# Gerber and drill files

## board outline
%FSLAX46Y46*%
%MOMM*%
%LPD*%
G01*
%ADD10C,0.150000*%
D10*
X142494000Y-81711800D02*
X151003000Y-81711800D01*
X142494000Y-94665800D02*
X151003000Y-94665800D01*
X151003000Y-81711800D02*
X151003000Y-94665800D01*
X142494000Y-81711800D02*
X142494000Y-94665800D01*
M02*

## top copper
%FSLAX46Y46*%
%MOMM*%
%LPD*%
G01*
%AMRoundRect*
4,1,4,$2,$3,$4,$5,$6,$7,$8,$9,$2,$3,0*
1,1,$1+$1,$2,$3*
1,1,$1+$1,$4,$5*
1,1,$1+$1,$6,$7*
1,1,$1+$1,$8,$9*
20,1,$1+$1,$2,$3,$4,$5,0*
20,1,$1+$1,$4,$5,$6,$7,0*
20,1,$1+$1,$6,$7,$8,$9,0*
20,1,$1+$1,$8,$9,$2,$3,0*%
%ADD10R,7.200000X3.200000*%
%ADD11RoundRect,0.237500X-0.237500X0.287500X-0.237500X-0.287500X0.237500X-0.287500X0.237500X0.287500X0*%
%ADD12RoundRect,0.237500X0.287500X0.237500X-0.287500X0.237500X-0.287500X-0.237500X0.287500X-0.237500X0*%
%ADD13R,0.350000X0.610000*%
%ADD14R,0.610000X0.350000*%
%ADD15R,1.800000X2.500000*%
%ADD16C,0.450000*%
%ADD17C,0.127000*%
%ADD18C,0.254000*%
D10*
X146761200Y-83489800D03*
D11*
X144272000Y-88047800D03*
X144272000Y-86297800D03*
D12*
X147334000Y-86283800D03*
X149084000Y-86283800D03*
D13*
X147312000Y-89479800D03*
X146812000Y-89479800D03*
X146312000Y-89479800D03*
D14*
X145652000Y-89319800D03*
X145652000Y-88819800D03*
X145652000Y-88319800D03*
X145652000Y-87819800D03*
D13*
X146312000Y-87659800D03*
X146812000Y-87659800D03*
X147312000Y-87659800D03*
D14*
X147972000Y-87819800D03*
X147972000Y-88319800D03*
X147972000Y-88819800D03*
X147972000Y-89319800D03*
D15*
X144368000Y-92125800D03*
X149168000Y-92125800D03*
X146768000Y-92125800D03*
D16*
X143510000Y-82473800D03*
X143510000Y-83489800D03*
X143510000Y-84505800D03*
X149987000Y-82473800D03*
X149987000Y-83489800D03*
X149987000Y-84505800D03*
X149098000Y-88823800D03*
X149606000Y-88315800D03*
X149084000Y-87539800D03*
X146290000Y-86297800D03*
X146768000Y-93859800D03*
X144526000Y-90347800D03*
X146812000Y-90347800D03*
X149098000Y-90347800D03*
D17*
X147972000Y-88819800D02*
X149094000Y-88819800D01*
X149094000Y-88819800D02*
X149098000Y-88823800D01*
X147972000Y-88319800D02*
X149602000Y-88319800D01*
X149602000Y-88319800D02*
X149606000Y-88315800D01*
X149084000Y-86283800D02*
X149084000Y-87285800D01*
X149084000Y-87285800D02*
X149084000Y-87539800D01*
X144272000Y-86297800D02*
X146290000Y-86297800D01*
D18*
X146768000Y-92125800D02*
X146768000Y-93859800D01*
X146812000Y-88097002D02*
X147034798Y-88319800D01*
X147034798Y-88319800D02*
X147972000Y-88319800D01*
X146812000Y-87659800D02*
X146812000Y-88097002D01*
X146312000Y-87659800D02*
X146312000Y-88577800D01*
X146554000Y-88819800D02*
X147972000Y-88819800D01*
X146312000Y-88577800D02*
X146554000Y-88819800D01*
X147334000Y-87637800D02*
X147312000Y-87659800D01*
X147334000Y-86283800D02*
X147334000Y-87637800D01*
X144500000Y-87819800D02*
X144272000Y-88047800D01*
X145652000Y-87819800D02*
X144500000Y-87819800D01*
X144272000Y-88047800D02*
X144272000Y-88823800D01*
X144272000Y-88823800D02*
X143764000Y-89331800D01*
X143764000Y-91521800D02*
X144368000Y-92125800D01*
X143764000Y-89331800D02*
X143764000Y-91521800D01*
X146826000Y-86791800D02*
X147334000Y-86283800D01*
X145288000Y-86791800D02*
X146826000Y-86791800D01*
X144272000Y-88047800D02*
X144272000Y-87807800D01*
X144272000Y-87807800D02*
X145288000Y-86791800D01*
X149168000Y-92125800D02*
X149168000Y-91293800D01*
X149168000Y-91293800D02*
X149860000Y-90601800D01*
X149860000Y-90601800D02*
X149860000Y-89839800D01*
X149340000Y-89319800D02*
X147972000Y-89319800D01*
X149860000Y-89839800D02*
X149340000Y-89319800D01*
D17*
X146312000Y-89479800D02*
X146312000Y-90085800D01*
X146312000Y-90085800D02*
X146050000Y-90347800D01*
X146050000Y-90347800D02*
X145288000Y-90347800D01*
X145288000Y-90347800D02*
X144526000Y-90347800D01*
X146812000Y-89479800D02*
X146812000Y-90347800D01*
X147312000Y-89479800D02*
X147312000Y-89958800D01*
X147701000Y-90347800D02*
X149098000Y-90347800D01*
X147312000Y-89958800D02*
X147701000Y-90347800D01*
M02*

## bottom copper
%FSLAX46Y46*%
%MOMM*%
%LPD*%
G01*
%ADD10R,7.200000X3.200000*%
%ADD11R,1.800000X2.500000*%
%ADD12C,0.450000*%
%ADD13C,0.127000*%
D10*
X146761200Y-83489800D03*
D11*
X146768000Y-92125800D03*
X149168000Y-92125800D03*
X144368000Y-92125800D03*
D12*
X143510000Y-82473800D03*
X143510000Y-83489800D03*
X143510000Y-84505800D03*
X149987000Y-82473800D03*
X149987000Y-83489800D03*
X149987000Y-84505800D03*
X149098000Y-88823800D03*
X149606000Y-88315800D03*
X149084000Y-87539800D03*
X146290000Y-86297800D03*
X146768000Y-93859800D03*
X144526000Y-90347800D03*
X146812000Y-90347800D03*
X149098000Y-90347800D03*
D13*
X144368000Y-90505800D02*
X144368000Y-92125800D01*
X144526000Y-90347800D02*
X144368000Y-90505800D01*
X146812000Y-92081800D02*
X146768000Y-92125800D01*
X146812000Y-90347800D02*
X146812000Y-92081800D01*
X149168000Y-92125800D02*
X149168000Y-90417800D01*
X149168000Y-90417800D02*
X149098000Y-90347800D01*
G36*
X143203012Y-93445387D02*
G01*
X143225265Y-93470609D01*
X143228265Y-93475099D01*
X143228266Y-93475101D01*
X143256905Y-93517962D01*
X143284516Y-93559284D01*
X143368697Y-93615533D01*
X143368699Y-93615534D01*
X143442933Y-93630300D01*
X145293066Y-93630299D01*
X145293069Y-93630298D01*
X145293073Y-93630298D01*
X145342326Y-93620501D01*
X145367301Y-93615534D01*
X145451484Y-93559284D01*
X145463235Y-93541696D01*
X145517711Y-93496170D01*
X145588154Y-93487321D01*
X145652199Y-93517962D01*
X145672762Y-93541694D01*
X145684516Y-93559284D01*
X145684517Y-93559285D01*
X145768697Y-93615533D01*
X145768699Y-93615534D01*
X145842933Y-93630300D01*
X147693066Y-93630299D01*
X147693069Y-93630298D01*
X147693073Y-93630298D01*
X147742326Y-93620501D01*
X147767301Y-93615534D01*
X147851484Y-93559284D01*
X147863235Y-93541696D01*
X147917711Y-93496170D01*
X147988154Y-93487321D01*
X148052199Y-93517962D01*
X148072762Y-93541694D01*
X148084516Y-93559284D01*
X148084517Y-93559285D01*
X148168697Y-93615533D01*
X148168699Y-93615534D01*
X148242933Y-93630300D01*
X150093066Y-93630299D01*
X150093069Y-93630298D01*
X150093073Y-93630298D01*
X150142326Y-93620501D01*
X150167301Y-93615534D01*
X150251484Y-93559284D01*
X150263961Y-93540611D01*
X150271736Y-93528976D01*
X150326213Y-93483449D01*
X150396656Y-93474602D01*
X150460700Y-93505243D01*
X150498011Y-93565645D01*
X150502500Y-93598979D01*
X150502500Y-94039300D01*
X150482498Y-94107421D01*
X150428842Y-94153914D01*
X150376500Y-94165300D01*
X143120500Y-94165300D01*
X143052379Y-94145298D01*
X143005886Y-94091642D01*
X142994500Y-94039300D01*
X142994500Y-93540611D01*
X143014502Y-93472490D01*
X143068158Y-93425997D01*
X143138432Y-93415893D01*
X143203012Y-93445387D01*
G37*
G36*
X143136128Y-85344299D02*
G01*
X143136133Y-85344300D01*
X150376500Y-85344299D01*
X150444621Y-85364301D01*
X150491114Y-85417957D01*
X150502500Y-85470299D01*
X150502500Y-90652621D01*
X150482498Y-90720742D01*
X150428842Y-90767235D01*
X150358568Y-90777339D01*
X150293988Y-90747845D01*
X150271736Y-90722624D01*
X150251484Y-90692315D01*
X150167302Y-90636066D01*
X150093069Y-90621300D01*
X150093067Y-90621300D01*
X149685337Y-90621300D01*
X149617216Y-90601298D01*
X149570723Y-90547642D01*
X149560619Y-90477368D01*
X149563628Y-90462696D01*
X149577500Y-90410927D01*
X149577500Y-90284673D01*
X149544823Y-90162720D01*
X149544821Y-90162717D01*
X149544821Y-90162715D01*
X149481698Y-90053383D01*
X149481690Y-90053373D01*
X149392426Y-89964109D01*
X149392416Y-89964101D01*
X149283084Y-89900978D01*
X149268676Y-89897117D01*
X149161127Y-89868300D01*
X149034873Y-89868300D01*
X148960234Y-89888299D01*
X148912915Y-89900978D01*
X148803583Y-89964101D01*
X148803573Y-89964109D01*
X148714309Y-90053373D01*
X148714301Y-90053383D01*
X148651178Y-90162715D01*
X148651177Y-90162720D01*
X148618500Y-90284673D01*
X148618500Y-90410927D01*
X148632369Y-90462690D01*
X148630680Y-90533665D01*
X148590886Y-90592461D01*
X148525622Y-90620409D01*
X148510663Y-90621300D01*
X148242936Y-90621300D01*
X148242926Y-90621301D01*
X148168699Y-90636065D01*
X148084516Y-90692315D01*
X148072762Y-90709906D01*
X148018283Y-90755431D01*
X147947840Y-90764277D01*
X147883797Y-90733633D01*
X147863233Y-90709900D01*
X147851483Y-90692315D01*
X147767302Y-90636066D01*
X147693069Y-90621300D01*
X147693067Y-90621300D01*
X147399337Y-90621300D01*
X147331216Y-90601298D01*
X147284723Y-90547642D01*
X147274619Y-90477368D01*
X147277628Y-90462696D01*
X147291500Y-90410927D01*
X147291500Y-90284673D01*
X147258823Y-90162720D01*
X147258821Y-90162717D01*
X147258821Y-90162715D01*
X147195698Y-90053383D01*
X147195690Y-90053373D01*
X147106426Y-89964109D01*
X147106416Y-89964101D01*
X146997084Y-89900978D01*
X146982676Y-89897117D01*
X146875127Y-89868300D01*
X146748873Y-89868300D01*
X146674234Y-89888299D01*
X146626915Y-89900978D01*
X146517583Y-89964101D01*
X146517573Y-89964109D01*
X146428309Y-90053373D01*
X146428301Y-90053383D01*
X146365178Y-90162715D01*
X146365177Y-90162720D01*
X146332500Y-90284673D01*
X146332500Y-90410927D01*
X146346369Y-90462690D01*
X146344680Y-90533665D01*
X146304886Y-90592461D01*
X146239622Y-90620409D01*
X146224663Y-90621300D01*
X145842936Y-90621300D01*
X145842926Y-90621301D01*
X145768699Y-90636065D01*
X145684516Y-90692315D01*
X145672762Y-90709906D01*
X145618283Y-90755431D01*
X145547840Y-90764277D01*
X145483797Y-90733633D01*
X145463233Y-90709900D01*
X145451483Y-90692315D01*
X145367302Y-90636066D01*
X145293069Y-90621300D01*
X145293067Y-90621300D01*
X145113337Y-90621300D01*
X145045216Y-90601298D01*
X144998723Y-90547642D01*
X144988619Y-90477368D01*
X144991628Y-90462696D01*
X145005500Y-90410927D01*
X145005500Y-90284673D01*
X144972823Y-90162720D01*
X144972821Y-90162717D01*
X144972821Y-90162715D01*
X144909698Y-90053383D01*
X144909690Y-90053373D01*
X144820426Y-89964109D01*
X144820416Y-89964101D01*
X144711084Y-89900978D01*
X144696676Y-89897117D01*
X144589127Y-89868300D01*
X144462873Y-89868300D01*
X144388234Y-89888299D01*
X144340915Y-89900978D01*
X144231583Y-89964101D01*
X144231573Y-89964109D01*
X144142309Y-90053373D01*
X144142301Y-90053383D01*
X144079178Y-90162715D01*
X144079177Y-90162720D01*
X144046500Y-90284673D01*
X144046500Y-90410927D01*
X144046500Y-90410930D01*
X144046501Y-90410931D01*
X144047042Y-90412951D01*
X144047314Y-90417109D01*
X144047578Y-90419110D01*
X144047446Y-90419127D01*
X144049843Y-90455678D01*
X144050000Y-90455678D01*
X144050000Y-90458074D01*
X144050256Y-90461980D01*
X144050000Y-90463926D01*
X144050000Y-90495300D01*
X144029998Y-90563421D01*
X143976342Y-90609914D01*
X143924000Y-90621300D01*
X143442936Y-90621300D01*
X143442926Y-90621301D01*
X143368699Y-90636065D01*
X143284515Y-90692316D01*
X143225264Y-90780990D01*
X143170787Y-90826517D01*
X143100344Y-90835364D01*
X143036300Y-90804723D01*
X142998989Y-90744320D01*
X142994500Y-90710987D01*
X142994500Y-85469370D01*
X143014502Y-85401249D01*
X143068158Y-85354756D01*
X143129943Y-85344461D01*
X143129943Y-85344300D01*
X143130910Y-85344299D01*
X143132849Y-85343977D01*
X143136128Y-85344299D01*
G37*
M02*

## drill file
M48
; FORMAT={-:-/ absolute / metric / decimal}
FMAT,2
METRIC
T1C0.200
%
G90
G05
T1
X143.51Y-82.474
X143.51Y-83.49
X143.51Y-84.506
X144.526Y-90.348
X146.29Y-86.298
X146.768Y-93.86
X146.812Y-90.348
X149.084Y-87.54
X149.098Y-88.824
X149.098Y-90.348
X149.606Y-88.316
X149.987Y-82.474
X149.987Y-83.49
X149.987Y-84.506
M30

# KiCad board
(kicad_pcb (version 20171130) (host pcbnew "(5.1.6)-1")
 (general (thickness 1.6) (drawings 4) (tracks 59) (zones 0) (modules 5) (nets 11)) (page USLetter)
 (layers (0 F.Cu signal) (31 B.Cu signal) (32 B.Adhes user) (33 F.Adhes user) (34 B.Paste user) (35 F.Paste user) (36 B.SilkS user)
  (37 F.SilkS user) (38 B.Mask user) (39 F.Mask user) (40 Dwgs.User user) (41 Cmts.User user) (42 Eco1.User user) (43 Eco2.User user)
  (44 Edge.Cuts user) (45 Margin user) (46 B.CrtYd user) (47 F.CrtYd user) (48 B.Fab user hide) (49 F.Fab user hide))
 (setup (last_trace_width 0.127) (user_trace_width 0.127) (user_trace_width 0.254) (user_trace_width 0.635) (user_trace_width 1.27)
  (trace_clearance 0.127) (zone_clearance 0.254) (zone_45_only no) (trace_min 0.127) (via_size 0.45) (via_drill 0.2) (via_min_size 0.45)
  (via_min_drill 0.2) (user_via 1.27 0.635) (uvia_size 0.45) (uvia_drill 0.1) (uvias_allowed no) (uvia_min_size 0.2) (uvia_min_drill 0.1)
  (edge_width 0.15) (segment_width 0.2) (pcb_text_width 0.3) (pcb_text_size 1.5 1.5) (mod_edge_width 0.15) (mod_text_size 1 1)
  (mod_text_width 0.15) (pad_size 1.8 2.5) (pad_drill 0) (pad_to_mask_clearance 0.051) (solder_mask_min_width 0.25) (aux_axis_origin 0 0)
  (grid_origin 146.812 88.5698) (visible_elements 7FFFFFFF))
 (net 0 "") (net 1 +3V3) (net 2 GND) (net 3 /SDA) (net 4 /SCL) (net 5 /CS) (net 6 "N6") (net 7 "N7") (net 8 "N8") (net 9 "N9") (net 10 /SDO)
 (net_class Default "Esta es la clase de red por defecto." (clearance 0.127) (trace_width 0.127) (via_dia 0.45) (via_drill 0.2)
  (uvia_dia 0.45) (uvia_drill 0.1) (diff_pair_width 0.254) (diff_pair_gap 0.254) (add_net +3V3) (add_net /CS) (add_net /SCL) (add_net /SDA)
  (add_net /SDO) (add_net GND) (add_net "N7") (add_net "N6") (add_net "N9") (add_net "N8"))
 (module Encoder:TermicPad (layer F.Cu) (at 146.7612 83.4898)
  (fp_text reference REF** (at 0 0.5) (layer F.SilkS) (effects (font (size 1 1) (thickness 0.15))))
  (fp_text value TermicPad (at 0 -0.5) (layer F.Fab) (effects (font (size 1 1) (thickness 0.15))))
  (pad 1 smd rect (at 0 0) (size 7.2 3.2) (layers B.Cu B.Mask))
  (pad 1 smd rect (at 0 0) (size 7.2 3.2) (layers F.Cu F.Mask)))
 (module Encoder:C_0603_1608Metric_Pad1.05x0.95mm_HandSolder (layer F.Cu) (at 144.272 87.1728 270)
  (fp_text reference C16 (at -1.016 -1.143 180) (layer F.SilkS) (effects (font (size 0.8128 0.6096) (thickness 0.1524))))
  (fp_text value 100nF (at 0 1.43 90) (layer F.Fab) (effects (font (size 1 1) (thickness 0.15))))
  (pad 2 smd roundrect (at 0.875 0 270) (size 1.05 0.95) (layers F.Cu F.Paste F.Mask) (roundrect_rratio 0.25) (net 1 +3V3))
  (pad 1 smd roundrect (at -0.875 0 270) (size 1.05 0.95) (layers F.Cu F.Paste F.Mask) (roundrect_rratio 0.25) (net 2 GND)))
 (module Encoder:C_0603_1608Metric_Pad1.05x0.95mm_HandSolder (layer F.Cu) (at 148.209 86.2838 180)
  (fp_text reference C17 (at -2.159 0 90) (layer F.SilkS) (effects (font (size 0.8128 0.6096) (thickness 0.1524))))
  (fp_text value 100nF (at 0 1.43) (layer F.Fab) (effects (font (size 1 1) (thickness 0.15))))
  (pad 2 smd roundrect (at 0.875 0 180) (size 1.05 0.95) (layers F.Cu F.Paste F.Mask) (roundrect_rratio 0.25) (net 1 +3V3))
  (pad 1 smd roundrect (at -0.875 0 180) (size 1.05 0.95) (layers F.Cu F.Paste F.Mask) (roundrect_rratio 0.25) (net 2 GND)))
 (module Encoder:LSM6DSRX (layer F.Cu) (at 146.812 88.5698 180)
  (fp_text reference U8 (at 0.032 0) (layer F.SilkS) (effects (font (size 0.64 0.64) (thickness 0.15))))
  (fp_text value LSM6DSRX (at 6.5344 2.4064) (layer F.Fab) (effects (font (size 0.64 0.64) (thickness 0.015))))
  (pad 14 smd rect (at -0.5 -0.91 180) (size 0.35 0.61) (layers F.Cu F.Paste F.Mask) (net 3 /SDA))
  (pad 13 smd rect (at 0 -0.91 180) (size 0.35 0.61) (layers F.Cu F.Paste F.Mask) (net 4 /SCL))
  (pad 12 smd rect (at 0.5 -0.91 180) (size 0.35 0.61) (layers F.Cu F.Paste F.Mask) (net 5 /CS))
  (pad 11 smd rect (at 1.16 -0.75 180) (size 0.61 0.35) (layers F.Cu F.Paste F.Mask) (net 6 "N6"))
  (pad 10 smd rect (at 1.16 -0.25 180) (size 0.61 0.35) (layers F.Cu F.Paste F.Mask) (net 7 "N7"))
  (pad 9 smd rect (at 1.16 0.25 180) (size 0.61 0.35) (layers F.Cu F.Paste F.Mask) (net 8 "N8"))
  (pad 8 smd rect (at 1.16 0.75 180) (size 0.61 0.35) (layers F.Cu F.Paste F.Mask) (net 1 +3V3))
  (pad 7 smd rect (at 0.5 0.91 180) (size 0.35 0.61) (layers F.Cu F.Paste F.Mask) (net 2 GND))
  (pad 6 smd rect (at 0 0.91 180) (size 0.35 0.61) (layers F.Cu F.Paste F.Mask) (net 2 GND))
  (pad 5 smd rect (at -0.5 0.91 180) (size 0.35 0.61) (layers F.Cu F.Paste F.Mask) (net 1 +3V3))
  (pad 4 smd rect (at -1.16 0.75 180) (size 0.61 0.35) (layers F.Cu F.Paste F.Mask) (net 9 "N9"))
  (pad 3 smd rect (at -1.16 0.25 180) (size 0.61 0.35) (layers F.Cu F.Paste F.Mask) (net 2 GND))
  (pad 2 smd rect (at -1.16 -0.25 180) (size 0.61 0.35) (layers F.Cu F.Paste F.Mask) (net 2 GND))
  (pad 1 smd rect (at -1.16 -0.75 180) (size 0.61 0.35) (layers F.Cu F.Paste F.Mask) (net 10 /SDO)))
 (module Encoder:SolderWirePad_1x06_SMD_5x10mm (layer F.Cu) (at 146.812 92.1258)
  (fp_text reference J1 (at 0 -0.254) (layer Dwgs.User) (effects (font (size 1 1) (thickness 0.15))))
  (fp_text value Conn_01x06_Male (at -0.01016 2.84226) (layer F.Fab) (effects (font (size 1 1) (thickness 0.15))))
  (pad 2 smd rect (at -0.044 0) (size 1.8 2.5) (layers B.Cu B.Paste B.Mask) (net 4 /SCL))
  (pad 3 smd rect (at 2.356 0) (size 1.8 2.5) (layers B.Cu B.Paste B.Mask) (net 3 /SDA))
  (pad 6 smd rect (at -2.444 0) (size 1.8 2.5) (layers F.Cu F.Paste F.Mask) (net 1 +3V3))
  (pad 4 smd rect (at 2.356 0) (size 1.8 2.5) (layers F.Cu F.Paste F.Mask) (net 10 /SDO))
  (pad 1 smd rect (at -2.444 0) (size 1.8 2.5) (layers B.Cu B.Paste B.Mask) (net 5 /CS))
  (pad 5 smd rect (at -0.044 0) (size 1.8 2.5) (layers F.Cu F.Paste F.Mask) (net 2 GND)))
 (gr_line (start 142.494 81.7118) (end 151.003 81.7118) (layer Edge.Cuts) (width 0.15))
 (gr_line (start 142.494 94.6658) (end 151.003 94.6658) (layer Edge.Cuts) (width 0.15))
 (gr_line (start 151.003 81.7118) (end 151.003 94.6658) (layer Edge.Cuts) (width 0.15))
 (gr_line (start 142.494 81.7118) (end 142.494 94.6658) (layer Edge.Cuts) (width 0.15))
 (via (at 143.51 82.4738) (size 0.45) (drill 0.2) (layers F.Cu B.Cu) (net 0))
 (via (at 143.51 83.4898) (size 0.45) (drill 0.2) (layers F.Cu B.Cu) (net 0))
 (via (at 143.51 84.5058) (size 0.45) (drill 0.2) (layers F.Cu B.Cu) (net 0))
 (via (at 149.987 82.4738) (size 0.45) (drill 0.2) (layers F.Cu B.Cu) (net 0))
 (via (at 149.987 83.4898) (size 0.45) (drill 0.2) (layers F.Cu B.Cu) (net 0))
 (via (at 149.987 84.5058) (size 0.45) (drill 0.2) (layers F.Cu B.Cu) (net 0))
 (segment (start 147.972 88.8198) (end 149.094 88.8198) (width 0.127) (layer F.Cu) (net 2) (status 10))
 (via (at 149.098 88.8238) (size 0.45) (drill 0.2) (layers F.Cu B.Cu) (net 2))
 (segment (start 149.094 88.8198) (end 149.098 88.8238) (width 0.127) (layer F.Cu) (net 2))
 (segment (start 147.972 88.3198) (end 149.602 88.3198) (width 0.127) (layer F.Cu) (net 2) (status 10))
 (via (at 149.606 88.3158) (size 0.45) (drill 0.2) (layers F.Cu B.Cu) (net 2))
 (segment (start 149.602 88.3198) (end 149.606 88.3158) (width 0.127) (layer F.Cu) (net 2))
 (segment (start 149.084 86.2838) (end 149.084 87.2858) (width 0.127) (layer F.Cu) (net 2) (status 10))
 (segment (start 149.084 87.2858) (end 149.084 87.5398) (width 0.127) (layer F.Cu) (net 2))
 (via (at 149.084 87.5398) (size 0.45) (drill 0.2) (layers F.Cu B.Cu) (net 2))
 (segment (start 144.272 86.2978) (end 146.29 86.2978) (width 0.127) (layer F.Cu) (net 2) (status 10))
 (via (at 146.29 86.2978) (size 0.45) (drill 0.2) (layers F.Cu B.Cu) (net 2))
 (segment (start 146.768 92.1258) (end 146.768 93.8598) (width 0.254) (layer F.Cu) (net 2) (status 10))
 (via (at 146.768 93.8598) (size 0.45) (drill 0.2) (layers F.Cu B.Cu) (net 2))
 (segment (start 146.812 88.097002) (end 147.034798 88.3198) (width 0.254) (layer F.Cu) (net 2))
 (segment (start 147.034798 88.3198) (end 147.972 88.3198) (width 0.254) (layer F.Cu) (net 2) (status 20))
 (segment (start 146.812 87.6598) (end 146.812 88.097002) (width 0.254) (layer F.Cu) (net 2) (status 10))
 (segment (start 146.312 87.6598) (end 146.312 88.5778) (width 0.254) (layer F.Cu) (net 2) (status 10))
 (segment (start 146.554 88.8198) (end 147.972 88.8198) (width 0.254) (layer F.Cu) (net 2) (status 20))
 (segment (start 146.312 88.5778) (end 146.554 88.8198) (width 0.254) (layer F.Cu) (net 2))
 (segment (start 147.334 87.6378) (end 147.312 87.6598) (width 0.254) (layer F.Cu) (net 1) (status 30))
 (segment (start 147.334 86.2838) (end 147.334 87.6378) (width 0.254) (layer F.Cu) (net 1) (status 30))
 (segment (start 144.5 87.8198) (end 144.272 88.0478) (width 0.254) (layer F.Cu) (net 1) (status 30))
 (segment (start 145.652 87.8198) (end 144.5 87.8198) (width 0.254) (layer F.Cu) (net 1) (status 30))
 (segment (start 144.272 88.0478) (end 144.272 88.8238) (width 0.254) (layer F.Cu) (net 1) (status 10))
 (segment (start 144.272 88.8238) (end 143.764 89.3318) (width 0.254) (layer F.Cu) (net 1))
 (segment (start 143.764 91.5218) (end 144.368 92.1258) (width 0.254) (layer F.Cu) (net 1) (status 30))
 (segment (start 143.764 89.3318) (end 143.764 91.5218) (width 0.254) (layer F.Cu) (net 1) (status 20))
 (segment (start 146.826 86.7918) (end 147.334 86.2838) (width 0.254) (layer F.Cu) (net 1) (status 20))
 (segment (start 145.288 86.7918) (end 146.826 86.7918) (width 0.254) (layer F.Cu) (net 1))
 (segment (start 144.272 88.0478) (end 144.272 87.8078) (width 0.254) (layer F.Cu) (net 1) (status 30))
 (segment (start 144.272 87.8078) (end 145.288 86.7918) (width 0.254) (layer F.Cu) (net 1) (status 10))
 (segment (start 149.168 92.1258) (end 149.168 91.2938) (width 0.254) (layer F.Cu) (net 10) (status 30))
 (segment (start 149.168 91.2938) (end 149.86 90.6018) (width 0.254) (layer F.Cu) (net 10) (status 10))
 (segment (start 149.86 90.6018) (end 149.86 89.8398) (width 0.254) (layer F.Cu) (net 10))
 (segment (start 149.34 89.3198) (end 147.972 89.3198) (width 0.254) (layer F.Cu) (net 10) (status 20))
 (segment (start 149.86 89.8398) (end 149.34 89.3198) (width 0.254) (layer F.Cu) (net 10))
 (segment (start 146.312 89.4798) (end 146.312 90.0858) (width 0.127) (layer F.Cu) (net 5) (status 10))
 (segment (start 146.312 90.0858) (end 146.05 90.3478) (width 0.127) (layer F.Cu) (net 5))
 (segment (start 146.05 90.3478) (end 145.288 90.3478) (width 0.127) (layer F.Cu) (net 5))
 (segment (start 145.288 90.3478) (end 144.526 90.3478) (width 0.127) (layer F.Cu) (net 5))
 (via (at 144.526 90.3478) (size 0.45) (drill 0.2) (layers F.Cu B.Cu) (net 5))
 (segment (start 144.368 90.5058) (end 144.368 92.1258) (width 0.127) (layer B.Cu) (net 5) (status 20))
 (segment (start 144.526 90.3478) (end 144.368 90.5058) (width 0.127) (layer B.Cu) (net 5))
 (segment (start 146.812 89.4798) (end 146.812 90.3478) (width 0.127) (layer F.Cu) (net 4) (status 10))
 (via (at 146.812 90.3478) (size 0.45) (drill 0.2) (layers F.Cu B.Cu) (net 4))
 (segment (start 146.812 92.0818) (end 146.768 92.1258) (width 0.127) (layer B.Cu) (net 4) (status 30))
 (segment (start 146.812 90.3478) (end 146.812 92.0818) (width 0.127) (layer B.Cu) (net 4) (status 20))
 (segment (start 149.168 92.1258) (end 149.168 90.4178) (width 0.127) (layer B.Cu) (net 3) (status 10))
 (via (at 149.098 90.3478) (size 0.45) (drill 0.2) (layers F.Cu B.Cu) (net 3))
 (segment (start 149.168 90.4178) (end 149.098 90.3478) (width 0.127) (layer B.Cu) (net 3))
 (segment (start 147.312 89.4798) (end 147.312 89.9588) (width 0.127) (layer F.Cu) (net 3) (status 10))
 (segment (start 147.701 90.3478) (end 149.098 90.3478) (width 0.127) (layer F.Cu) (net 3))
 (segment (start 147.312 89.9588) (end 147.701 90.3478) (width 0.127) (layer F.Cu) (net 3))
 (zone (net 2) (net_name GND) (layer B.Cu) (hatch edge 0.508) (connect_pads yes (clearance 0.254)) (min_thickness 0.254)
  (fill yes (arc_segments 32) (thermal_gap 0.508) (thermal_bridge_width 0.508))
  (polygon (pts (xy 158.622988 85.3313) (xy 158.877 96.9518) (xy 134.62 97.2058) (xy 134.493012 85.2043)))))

